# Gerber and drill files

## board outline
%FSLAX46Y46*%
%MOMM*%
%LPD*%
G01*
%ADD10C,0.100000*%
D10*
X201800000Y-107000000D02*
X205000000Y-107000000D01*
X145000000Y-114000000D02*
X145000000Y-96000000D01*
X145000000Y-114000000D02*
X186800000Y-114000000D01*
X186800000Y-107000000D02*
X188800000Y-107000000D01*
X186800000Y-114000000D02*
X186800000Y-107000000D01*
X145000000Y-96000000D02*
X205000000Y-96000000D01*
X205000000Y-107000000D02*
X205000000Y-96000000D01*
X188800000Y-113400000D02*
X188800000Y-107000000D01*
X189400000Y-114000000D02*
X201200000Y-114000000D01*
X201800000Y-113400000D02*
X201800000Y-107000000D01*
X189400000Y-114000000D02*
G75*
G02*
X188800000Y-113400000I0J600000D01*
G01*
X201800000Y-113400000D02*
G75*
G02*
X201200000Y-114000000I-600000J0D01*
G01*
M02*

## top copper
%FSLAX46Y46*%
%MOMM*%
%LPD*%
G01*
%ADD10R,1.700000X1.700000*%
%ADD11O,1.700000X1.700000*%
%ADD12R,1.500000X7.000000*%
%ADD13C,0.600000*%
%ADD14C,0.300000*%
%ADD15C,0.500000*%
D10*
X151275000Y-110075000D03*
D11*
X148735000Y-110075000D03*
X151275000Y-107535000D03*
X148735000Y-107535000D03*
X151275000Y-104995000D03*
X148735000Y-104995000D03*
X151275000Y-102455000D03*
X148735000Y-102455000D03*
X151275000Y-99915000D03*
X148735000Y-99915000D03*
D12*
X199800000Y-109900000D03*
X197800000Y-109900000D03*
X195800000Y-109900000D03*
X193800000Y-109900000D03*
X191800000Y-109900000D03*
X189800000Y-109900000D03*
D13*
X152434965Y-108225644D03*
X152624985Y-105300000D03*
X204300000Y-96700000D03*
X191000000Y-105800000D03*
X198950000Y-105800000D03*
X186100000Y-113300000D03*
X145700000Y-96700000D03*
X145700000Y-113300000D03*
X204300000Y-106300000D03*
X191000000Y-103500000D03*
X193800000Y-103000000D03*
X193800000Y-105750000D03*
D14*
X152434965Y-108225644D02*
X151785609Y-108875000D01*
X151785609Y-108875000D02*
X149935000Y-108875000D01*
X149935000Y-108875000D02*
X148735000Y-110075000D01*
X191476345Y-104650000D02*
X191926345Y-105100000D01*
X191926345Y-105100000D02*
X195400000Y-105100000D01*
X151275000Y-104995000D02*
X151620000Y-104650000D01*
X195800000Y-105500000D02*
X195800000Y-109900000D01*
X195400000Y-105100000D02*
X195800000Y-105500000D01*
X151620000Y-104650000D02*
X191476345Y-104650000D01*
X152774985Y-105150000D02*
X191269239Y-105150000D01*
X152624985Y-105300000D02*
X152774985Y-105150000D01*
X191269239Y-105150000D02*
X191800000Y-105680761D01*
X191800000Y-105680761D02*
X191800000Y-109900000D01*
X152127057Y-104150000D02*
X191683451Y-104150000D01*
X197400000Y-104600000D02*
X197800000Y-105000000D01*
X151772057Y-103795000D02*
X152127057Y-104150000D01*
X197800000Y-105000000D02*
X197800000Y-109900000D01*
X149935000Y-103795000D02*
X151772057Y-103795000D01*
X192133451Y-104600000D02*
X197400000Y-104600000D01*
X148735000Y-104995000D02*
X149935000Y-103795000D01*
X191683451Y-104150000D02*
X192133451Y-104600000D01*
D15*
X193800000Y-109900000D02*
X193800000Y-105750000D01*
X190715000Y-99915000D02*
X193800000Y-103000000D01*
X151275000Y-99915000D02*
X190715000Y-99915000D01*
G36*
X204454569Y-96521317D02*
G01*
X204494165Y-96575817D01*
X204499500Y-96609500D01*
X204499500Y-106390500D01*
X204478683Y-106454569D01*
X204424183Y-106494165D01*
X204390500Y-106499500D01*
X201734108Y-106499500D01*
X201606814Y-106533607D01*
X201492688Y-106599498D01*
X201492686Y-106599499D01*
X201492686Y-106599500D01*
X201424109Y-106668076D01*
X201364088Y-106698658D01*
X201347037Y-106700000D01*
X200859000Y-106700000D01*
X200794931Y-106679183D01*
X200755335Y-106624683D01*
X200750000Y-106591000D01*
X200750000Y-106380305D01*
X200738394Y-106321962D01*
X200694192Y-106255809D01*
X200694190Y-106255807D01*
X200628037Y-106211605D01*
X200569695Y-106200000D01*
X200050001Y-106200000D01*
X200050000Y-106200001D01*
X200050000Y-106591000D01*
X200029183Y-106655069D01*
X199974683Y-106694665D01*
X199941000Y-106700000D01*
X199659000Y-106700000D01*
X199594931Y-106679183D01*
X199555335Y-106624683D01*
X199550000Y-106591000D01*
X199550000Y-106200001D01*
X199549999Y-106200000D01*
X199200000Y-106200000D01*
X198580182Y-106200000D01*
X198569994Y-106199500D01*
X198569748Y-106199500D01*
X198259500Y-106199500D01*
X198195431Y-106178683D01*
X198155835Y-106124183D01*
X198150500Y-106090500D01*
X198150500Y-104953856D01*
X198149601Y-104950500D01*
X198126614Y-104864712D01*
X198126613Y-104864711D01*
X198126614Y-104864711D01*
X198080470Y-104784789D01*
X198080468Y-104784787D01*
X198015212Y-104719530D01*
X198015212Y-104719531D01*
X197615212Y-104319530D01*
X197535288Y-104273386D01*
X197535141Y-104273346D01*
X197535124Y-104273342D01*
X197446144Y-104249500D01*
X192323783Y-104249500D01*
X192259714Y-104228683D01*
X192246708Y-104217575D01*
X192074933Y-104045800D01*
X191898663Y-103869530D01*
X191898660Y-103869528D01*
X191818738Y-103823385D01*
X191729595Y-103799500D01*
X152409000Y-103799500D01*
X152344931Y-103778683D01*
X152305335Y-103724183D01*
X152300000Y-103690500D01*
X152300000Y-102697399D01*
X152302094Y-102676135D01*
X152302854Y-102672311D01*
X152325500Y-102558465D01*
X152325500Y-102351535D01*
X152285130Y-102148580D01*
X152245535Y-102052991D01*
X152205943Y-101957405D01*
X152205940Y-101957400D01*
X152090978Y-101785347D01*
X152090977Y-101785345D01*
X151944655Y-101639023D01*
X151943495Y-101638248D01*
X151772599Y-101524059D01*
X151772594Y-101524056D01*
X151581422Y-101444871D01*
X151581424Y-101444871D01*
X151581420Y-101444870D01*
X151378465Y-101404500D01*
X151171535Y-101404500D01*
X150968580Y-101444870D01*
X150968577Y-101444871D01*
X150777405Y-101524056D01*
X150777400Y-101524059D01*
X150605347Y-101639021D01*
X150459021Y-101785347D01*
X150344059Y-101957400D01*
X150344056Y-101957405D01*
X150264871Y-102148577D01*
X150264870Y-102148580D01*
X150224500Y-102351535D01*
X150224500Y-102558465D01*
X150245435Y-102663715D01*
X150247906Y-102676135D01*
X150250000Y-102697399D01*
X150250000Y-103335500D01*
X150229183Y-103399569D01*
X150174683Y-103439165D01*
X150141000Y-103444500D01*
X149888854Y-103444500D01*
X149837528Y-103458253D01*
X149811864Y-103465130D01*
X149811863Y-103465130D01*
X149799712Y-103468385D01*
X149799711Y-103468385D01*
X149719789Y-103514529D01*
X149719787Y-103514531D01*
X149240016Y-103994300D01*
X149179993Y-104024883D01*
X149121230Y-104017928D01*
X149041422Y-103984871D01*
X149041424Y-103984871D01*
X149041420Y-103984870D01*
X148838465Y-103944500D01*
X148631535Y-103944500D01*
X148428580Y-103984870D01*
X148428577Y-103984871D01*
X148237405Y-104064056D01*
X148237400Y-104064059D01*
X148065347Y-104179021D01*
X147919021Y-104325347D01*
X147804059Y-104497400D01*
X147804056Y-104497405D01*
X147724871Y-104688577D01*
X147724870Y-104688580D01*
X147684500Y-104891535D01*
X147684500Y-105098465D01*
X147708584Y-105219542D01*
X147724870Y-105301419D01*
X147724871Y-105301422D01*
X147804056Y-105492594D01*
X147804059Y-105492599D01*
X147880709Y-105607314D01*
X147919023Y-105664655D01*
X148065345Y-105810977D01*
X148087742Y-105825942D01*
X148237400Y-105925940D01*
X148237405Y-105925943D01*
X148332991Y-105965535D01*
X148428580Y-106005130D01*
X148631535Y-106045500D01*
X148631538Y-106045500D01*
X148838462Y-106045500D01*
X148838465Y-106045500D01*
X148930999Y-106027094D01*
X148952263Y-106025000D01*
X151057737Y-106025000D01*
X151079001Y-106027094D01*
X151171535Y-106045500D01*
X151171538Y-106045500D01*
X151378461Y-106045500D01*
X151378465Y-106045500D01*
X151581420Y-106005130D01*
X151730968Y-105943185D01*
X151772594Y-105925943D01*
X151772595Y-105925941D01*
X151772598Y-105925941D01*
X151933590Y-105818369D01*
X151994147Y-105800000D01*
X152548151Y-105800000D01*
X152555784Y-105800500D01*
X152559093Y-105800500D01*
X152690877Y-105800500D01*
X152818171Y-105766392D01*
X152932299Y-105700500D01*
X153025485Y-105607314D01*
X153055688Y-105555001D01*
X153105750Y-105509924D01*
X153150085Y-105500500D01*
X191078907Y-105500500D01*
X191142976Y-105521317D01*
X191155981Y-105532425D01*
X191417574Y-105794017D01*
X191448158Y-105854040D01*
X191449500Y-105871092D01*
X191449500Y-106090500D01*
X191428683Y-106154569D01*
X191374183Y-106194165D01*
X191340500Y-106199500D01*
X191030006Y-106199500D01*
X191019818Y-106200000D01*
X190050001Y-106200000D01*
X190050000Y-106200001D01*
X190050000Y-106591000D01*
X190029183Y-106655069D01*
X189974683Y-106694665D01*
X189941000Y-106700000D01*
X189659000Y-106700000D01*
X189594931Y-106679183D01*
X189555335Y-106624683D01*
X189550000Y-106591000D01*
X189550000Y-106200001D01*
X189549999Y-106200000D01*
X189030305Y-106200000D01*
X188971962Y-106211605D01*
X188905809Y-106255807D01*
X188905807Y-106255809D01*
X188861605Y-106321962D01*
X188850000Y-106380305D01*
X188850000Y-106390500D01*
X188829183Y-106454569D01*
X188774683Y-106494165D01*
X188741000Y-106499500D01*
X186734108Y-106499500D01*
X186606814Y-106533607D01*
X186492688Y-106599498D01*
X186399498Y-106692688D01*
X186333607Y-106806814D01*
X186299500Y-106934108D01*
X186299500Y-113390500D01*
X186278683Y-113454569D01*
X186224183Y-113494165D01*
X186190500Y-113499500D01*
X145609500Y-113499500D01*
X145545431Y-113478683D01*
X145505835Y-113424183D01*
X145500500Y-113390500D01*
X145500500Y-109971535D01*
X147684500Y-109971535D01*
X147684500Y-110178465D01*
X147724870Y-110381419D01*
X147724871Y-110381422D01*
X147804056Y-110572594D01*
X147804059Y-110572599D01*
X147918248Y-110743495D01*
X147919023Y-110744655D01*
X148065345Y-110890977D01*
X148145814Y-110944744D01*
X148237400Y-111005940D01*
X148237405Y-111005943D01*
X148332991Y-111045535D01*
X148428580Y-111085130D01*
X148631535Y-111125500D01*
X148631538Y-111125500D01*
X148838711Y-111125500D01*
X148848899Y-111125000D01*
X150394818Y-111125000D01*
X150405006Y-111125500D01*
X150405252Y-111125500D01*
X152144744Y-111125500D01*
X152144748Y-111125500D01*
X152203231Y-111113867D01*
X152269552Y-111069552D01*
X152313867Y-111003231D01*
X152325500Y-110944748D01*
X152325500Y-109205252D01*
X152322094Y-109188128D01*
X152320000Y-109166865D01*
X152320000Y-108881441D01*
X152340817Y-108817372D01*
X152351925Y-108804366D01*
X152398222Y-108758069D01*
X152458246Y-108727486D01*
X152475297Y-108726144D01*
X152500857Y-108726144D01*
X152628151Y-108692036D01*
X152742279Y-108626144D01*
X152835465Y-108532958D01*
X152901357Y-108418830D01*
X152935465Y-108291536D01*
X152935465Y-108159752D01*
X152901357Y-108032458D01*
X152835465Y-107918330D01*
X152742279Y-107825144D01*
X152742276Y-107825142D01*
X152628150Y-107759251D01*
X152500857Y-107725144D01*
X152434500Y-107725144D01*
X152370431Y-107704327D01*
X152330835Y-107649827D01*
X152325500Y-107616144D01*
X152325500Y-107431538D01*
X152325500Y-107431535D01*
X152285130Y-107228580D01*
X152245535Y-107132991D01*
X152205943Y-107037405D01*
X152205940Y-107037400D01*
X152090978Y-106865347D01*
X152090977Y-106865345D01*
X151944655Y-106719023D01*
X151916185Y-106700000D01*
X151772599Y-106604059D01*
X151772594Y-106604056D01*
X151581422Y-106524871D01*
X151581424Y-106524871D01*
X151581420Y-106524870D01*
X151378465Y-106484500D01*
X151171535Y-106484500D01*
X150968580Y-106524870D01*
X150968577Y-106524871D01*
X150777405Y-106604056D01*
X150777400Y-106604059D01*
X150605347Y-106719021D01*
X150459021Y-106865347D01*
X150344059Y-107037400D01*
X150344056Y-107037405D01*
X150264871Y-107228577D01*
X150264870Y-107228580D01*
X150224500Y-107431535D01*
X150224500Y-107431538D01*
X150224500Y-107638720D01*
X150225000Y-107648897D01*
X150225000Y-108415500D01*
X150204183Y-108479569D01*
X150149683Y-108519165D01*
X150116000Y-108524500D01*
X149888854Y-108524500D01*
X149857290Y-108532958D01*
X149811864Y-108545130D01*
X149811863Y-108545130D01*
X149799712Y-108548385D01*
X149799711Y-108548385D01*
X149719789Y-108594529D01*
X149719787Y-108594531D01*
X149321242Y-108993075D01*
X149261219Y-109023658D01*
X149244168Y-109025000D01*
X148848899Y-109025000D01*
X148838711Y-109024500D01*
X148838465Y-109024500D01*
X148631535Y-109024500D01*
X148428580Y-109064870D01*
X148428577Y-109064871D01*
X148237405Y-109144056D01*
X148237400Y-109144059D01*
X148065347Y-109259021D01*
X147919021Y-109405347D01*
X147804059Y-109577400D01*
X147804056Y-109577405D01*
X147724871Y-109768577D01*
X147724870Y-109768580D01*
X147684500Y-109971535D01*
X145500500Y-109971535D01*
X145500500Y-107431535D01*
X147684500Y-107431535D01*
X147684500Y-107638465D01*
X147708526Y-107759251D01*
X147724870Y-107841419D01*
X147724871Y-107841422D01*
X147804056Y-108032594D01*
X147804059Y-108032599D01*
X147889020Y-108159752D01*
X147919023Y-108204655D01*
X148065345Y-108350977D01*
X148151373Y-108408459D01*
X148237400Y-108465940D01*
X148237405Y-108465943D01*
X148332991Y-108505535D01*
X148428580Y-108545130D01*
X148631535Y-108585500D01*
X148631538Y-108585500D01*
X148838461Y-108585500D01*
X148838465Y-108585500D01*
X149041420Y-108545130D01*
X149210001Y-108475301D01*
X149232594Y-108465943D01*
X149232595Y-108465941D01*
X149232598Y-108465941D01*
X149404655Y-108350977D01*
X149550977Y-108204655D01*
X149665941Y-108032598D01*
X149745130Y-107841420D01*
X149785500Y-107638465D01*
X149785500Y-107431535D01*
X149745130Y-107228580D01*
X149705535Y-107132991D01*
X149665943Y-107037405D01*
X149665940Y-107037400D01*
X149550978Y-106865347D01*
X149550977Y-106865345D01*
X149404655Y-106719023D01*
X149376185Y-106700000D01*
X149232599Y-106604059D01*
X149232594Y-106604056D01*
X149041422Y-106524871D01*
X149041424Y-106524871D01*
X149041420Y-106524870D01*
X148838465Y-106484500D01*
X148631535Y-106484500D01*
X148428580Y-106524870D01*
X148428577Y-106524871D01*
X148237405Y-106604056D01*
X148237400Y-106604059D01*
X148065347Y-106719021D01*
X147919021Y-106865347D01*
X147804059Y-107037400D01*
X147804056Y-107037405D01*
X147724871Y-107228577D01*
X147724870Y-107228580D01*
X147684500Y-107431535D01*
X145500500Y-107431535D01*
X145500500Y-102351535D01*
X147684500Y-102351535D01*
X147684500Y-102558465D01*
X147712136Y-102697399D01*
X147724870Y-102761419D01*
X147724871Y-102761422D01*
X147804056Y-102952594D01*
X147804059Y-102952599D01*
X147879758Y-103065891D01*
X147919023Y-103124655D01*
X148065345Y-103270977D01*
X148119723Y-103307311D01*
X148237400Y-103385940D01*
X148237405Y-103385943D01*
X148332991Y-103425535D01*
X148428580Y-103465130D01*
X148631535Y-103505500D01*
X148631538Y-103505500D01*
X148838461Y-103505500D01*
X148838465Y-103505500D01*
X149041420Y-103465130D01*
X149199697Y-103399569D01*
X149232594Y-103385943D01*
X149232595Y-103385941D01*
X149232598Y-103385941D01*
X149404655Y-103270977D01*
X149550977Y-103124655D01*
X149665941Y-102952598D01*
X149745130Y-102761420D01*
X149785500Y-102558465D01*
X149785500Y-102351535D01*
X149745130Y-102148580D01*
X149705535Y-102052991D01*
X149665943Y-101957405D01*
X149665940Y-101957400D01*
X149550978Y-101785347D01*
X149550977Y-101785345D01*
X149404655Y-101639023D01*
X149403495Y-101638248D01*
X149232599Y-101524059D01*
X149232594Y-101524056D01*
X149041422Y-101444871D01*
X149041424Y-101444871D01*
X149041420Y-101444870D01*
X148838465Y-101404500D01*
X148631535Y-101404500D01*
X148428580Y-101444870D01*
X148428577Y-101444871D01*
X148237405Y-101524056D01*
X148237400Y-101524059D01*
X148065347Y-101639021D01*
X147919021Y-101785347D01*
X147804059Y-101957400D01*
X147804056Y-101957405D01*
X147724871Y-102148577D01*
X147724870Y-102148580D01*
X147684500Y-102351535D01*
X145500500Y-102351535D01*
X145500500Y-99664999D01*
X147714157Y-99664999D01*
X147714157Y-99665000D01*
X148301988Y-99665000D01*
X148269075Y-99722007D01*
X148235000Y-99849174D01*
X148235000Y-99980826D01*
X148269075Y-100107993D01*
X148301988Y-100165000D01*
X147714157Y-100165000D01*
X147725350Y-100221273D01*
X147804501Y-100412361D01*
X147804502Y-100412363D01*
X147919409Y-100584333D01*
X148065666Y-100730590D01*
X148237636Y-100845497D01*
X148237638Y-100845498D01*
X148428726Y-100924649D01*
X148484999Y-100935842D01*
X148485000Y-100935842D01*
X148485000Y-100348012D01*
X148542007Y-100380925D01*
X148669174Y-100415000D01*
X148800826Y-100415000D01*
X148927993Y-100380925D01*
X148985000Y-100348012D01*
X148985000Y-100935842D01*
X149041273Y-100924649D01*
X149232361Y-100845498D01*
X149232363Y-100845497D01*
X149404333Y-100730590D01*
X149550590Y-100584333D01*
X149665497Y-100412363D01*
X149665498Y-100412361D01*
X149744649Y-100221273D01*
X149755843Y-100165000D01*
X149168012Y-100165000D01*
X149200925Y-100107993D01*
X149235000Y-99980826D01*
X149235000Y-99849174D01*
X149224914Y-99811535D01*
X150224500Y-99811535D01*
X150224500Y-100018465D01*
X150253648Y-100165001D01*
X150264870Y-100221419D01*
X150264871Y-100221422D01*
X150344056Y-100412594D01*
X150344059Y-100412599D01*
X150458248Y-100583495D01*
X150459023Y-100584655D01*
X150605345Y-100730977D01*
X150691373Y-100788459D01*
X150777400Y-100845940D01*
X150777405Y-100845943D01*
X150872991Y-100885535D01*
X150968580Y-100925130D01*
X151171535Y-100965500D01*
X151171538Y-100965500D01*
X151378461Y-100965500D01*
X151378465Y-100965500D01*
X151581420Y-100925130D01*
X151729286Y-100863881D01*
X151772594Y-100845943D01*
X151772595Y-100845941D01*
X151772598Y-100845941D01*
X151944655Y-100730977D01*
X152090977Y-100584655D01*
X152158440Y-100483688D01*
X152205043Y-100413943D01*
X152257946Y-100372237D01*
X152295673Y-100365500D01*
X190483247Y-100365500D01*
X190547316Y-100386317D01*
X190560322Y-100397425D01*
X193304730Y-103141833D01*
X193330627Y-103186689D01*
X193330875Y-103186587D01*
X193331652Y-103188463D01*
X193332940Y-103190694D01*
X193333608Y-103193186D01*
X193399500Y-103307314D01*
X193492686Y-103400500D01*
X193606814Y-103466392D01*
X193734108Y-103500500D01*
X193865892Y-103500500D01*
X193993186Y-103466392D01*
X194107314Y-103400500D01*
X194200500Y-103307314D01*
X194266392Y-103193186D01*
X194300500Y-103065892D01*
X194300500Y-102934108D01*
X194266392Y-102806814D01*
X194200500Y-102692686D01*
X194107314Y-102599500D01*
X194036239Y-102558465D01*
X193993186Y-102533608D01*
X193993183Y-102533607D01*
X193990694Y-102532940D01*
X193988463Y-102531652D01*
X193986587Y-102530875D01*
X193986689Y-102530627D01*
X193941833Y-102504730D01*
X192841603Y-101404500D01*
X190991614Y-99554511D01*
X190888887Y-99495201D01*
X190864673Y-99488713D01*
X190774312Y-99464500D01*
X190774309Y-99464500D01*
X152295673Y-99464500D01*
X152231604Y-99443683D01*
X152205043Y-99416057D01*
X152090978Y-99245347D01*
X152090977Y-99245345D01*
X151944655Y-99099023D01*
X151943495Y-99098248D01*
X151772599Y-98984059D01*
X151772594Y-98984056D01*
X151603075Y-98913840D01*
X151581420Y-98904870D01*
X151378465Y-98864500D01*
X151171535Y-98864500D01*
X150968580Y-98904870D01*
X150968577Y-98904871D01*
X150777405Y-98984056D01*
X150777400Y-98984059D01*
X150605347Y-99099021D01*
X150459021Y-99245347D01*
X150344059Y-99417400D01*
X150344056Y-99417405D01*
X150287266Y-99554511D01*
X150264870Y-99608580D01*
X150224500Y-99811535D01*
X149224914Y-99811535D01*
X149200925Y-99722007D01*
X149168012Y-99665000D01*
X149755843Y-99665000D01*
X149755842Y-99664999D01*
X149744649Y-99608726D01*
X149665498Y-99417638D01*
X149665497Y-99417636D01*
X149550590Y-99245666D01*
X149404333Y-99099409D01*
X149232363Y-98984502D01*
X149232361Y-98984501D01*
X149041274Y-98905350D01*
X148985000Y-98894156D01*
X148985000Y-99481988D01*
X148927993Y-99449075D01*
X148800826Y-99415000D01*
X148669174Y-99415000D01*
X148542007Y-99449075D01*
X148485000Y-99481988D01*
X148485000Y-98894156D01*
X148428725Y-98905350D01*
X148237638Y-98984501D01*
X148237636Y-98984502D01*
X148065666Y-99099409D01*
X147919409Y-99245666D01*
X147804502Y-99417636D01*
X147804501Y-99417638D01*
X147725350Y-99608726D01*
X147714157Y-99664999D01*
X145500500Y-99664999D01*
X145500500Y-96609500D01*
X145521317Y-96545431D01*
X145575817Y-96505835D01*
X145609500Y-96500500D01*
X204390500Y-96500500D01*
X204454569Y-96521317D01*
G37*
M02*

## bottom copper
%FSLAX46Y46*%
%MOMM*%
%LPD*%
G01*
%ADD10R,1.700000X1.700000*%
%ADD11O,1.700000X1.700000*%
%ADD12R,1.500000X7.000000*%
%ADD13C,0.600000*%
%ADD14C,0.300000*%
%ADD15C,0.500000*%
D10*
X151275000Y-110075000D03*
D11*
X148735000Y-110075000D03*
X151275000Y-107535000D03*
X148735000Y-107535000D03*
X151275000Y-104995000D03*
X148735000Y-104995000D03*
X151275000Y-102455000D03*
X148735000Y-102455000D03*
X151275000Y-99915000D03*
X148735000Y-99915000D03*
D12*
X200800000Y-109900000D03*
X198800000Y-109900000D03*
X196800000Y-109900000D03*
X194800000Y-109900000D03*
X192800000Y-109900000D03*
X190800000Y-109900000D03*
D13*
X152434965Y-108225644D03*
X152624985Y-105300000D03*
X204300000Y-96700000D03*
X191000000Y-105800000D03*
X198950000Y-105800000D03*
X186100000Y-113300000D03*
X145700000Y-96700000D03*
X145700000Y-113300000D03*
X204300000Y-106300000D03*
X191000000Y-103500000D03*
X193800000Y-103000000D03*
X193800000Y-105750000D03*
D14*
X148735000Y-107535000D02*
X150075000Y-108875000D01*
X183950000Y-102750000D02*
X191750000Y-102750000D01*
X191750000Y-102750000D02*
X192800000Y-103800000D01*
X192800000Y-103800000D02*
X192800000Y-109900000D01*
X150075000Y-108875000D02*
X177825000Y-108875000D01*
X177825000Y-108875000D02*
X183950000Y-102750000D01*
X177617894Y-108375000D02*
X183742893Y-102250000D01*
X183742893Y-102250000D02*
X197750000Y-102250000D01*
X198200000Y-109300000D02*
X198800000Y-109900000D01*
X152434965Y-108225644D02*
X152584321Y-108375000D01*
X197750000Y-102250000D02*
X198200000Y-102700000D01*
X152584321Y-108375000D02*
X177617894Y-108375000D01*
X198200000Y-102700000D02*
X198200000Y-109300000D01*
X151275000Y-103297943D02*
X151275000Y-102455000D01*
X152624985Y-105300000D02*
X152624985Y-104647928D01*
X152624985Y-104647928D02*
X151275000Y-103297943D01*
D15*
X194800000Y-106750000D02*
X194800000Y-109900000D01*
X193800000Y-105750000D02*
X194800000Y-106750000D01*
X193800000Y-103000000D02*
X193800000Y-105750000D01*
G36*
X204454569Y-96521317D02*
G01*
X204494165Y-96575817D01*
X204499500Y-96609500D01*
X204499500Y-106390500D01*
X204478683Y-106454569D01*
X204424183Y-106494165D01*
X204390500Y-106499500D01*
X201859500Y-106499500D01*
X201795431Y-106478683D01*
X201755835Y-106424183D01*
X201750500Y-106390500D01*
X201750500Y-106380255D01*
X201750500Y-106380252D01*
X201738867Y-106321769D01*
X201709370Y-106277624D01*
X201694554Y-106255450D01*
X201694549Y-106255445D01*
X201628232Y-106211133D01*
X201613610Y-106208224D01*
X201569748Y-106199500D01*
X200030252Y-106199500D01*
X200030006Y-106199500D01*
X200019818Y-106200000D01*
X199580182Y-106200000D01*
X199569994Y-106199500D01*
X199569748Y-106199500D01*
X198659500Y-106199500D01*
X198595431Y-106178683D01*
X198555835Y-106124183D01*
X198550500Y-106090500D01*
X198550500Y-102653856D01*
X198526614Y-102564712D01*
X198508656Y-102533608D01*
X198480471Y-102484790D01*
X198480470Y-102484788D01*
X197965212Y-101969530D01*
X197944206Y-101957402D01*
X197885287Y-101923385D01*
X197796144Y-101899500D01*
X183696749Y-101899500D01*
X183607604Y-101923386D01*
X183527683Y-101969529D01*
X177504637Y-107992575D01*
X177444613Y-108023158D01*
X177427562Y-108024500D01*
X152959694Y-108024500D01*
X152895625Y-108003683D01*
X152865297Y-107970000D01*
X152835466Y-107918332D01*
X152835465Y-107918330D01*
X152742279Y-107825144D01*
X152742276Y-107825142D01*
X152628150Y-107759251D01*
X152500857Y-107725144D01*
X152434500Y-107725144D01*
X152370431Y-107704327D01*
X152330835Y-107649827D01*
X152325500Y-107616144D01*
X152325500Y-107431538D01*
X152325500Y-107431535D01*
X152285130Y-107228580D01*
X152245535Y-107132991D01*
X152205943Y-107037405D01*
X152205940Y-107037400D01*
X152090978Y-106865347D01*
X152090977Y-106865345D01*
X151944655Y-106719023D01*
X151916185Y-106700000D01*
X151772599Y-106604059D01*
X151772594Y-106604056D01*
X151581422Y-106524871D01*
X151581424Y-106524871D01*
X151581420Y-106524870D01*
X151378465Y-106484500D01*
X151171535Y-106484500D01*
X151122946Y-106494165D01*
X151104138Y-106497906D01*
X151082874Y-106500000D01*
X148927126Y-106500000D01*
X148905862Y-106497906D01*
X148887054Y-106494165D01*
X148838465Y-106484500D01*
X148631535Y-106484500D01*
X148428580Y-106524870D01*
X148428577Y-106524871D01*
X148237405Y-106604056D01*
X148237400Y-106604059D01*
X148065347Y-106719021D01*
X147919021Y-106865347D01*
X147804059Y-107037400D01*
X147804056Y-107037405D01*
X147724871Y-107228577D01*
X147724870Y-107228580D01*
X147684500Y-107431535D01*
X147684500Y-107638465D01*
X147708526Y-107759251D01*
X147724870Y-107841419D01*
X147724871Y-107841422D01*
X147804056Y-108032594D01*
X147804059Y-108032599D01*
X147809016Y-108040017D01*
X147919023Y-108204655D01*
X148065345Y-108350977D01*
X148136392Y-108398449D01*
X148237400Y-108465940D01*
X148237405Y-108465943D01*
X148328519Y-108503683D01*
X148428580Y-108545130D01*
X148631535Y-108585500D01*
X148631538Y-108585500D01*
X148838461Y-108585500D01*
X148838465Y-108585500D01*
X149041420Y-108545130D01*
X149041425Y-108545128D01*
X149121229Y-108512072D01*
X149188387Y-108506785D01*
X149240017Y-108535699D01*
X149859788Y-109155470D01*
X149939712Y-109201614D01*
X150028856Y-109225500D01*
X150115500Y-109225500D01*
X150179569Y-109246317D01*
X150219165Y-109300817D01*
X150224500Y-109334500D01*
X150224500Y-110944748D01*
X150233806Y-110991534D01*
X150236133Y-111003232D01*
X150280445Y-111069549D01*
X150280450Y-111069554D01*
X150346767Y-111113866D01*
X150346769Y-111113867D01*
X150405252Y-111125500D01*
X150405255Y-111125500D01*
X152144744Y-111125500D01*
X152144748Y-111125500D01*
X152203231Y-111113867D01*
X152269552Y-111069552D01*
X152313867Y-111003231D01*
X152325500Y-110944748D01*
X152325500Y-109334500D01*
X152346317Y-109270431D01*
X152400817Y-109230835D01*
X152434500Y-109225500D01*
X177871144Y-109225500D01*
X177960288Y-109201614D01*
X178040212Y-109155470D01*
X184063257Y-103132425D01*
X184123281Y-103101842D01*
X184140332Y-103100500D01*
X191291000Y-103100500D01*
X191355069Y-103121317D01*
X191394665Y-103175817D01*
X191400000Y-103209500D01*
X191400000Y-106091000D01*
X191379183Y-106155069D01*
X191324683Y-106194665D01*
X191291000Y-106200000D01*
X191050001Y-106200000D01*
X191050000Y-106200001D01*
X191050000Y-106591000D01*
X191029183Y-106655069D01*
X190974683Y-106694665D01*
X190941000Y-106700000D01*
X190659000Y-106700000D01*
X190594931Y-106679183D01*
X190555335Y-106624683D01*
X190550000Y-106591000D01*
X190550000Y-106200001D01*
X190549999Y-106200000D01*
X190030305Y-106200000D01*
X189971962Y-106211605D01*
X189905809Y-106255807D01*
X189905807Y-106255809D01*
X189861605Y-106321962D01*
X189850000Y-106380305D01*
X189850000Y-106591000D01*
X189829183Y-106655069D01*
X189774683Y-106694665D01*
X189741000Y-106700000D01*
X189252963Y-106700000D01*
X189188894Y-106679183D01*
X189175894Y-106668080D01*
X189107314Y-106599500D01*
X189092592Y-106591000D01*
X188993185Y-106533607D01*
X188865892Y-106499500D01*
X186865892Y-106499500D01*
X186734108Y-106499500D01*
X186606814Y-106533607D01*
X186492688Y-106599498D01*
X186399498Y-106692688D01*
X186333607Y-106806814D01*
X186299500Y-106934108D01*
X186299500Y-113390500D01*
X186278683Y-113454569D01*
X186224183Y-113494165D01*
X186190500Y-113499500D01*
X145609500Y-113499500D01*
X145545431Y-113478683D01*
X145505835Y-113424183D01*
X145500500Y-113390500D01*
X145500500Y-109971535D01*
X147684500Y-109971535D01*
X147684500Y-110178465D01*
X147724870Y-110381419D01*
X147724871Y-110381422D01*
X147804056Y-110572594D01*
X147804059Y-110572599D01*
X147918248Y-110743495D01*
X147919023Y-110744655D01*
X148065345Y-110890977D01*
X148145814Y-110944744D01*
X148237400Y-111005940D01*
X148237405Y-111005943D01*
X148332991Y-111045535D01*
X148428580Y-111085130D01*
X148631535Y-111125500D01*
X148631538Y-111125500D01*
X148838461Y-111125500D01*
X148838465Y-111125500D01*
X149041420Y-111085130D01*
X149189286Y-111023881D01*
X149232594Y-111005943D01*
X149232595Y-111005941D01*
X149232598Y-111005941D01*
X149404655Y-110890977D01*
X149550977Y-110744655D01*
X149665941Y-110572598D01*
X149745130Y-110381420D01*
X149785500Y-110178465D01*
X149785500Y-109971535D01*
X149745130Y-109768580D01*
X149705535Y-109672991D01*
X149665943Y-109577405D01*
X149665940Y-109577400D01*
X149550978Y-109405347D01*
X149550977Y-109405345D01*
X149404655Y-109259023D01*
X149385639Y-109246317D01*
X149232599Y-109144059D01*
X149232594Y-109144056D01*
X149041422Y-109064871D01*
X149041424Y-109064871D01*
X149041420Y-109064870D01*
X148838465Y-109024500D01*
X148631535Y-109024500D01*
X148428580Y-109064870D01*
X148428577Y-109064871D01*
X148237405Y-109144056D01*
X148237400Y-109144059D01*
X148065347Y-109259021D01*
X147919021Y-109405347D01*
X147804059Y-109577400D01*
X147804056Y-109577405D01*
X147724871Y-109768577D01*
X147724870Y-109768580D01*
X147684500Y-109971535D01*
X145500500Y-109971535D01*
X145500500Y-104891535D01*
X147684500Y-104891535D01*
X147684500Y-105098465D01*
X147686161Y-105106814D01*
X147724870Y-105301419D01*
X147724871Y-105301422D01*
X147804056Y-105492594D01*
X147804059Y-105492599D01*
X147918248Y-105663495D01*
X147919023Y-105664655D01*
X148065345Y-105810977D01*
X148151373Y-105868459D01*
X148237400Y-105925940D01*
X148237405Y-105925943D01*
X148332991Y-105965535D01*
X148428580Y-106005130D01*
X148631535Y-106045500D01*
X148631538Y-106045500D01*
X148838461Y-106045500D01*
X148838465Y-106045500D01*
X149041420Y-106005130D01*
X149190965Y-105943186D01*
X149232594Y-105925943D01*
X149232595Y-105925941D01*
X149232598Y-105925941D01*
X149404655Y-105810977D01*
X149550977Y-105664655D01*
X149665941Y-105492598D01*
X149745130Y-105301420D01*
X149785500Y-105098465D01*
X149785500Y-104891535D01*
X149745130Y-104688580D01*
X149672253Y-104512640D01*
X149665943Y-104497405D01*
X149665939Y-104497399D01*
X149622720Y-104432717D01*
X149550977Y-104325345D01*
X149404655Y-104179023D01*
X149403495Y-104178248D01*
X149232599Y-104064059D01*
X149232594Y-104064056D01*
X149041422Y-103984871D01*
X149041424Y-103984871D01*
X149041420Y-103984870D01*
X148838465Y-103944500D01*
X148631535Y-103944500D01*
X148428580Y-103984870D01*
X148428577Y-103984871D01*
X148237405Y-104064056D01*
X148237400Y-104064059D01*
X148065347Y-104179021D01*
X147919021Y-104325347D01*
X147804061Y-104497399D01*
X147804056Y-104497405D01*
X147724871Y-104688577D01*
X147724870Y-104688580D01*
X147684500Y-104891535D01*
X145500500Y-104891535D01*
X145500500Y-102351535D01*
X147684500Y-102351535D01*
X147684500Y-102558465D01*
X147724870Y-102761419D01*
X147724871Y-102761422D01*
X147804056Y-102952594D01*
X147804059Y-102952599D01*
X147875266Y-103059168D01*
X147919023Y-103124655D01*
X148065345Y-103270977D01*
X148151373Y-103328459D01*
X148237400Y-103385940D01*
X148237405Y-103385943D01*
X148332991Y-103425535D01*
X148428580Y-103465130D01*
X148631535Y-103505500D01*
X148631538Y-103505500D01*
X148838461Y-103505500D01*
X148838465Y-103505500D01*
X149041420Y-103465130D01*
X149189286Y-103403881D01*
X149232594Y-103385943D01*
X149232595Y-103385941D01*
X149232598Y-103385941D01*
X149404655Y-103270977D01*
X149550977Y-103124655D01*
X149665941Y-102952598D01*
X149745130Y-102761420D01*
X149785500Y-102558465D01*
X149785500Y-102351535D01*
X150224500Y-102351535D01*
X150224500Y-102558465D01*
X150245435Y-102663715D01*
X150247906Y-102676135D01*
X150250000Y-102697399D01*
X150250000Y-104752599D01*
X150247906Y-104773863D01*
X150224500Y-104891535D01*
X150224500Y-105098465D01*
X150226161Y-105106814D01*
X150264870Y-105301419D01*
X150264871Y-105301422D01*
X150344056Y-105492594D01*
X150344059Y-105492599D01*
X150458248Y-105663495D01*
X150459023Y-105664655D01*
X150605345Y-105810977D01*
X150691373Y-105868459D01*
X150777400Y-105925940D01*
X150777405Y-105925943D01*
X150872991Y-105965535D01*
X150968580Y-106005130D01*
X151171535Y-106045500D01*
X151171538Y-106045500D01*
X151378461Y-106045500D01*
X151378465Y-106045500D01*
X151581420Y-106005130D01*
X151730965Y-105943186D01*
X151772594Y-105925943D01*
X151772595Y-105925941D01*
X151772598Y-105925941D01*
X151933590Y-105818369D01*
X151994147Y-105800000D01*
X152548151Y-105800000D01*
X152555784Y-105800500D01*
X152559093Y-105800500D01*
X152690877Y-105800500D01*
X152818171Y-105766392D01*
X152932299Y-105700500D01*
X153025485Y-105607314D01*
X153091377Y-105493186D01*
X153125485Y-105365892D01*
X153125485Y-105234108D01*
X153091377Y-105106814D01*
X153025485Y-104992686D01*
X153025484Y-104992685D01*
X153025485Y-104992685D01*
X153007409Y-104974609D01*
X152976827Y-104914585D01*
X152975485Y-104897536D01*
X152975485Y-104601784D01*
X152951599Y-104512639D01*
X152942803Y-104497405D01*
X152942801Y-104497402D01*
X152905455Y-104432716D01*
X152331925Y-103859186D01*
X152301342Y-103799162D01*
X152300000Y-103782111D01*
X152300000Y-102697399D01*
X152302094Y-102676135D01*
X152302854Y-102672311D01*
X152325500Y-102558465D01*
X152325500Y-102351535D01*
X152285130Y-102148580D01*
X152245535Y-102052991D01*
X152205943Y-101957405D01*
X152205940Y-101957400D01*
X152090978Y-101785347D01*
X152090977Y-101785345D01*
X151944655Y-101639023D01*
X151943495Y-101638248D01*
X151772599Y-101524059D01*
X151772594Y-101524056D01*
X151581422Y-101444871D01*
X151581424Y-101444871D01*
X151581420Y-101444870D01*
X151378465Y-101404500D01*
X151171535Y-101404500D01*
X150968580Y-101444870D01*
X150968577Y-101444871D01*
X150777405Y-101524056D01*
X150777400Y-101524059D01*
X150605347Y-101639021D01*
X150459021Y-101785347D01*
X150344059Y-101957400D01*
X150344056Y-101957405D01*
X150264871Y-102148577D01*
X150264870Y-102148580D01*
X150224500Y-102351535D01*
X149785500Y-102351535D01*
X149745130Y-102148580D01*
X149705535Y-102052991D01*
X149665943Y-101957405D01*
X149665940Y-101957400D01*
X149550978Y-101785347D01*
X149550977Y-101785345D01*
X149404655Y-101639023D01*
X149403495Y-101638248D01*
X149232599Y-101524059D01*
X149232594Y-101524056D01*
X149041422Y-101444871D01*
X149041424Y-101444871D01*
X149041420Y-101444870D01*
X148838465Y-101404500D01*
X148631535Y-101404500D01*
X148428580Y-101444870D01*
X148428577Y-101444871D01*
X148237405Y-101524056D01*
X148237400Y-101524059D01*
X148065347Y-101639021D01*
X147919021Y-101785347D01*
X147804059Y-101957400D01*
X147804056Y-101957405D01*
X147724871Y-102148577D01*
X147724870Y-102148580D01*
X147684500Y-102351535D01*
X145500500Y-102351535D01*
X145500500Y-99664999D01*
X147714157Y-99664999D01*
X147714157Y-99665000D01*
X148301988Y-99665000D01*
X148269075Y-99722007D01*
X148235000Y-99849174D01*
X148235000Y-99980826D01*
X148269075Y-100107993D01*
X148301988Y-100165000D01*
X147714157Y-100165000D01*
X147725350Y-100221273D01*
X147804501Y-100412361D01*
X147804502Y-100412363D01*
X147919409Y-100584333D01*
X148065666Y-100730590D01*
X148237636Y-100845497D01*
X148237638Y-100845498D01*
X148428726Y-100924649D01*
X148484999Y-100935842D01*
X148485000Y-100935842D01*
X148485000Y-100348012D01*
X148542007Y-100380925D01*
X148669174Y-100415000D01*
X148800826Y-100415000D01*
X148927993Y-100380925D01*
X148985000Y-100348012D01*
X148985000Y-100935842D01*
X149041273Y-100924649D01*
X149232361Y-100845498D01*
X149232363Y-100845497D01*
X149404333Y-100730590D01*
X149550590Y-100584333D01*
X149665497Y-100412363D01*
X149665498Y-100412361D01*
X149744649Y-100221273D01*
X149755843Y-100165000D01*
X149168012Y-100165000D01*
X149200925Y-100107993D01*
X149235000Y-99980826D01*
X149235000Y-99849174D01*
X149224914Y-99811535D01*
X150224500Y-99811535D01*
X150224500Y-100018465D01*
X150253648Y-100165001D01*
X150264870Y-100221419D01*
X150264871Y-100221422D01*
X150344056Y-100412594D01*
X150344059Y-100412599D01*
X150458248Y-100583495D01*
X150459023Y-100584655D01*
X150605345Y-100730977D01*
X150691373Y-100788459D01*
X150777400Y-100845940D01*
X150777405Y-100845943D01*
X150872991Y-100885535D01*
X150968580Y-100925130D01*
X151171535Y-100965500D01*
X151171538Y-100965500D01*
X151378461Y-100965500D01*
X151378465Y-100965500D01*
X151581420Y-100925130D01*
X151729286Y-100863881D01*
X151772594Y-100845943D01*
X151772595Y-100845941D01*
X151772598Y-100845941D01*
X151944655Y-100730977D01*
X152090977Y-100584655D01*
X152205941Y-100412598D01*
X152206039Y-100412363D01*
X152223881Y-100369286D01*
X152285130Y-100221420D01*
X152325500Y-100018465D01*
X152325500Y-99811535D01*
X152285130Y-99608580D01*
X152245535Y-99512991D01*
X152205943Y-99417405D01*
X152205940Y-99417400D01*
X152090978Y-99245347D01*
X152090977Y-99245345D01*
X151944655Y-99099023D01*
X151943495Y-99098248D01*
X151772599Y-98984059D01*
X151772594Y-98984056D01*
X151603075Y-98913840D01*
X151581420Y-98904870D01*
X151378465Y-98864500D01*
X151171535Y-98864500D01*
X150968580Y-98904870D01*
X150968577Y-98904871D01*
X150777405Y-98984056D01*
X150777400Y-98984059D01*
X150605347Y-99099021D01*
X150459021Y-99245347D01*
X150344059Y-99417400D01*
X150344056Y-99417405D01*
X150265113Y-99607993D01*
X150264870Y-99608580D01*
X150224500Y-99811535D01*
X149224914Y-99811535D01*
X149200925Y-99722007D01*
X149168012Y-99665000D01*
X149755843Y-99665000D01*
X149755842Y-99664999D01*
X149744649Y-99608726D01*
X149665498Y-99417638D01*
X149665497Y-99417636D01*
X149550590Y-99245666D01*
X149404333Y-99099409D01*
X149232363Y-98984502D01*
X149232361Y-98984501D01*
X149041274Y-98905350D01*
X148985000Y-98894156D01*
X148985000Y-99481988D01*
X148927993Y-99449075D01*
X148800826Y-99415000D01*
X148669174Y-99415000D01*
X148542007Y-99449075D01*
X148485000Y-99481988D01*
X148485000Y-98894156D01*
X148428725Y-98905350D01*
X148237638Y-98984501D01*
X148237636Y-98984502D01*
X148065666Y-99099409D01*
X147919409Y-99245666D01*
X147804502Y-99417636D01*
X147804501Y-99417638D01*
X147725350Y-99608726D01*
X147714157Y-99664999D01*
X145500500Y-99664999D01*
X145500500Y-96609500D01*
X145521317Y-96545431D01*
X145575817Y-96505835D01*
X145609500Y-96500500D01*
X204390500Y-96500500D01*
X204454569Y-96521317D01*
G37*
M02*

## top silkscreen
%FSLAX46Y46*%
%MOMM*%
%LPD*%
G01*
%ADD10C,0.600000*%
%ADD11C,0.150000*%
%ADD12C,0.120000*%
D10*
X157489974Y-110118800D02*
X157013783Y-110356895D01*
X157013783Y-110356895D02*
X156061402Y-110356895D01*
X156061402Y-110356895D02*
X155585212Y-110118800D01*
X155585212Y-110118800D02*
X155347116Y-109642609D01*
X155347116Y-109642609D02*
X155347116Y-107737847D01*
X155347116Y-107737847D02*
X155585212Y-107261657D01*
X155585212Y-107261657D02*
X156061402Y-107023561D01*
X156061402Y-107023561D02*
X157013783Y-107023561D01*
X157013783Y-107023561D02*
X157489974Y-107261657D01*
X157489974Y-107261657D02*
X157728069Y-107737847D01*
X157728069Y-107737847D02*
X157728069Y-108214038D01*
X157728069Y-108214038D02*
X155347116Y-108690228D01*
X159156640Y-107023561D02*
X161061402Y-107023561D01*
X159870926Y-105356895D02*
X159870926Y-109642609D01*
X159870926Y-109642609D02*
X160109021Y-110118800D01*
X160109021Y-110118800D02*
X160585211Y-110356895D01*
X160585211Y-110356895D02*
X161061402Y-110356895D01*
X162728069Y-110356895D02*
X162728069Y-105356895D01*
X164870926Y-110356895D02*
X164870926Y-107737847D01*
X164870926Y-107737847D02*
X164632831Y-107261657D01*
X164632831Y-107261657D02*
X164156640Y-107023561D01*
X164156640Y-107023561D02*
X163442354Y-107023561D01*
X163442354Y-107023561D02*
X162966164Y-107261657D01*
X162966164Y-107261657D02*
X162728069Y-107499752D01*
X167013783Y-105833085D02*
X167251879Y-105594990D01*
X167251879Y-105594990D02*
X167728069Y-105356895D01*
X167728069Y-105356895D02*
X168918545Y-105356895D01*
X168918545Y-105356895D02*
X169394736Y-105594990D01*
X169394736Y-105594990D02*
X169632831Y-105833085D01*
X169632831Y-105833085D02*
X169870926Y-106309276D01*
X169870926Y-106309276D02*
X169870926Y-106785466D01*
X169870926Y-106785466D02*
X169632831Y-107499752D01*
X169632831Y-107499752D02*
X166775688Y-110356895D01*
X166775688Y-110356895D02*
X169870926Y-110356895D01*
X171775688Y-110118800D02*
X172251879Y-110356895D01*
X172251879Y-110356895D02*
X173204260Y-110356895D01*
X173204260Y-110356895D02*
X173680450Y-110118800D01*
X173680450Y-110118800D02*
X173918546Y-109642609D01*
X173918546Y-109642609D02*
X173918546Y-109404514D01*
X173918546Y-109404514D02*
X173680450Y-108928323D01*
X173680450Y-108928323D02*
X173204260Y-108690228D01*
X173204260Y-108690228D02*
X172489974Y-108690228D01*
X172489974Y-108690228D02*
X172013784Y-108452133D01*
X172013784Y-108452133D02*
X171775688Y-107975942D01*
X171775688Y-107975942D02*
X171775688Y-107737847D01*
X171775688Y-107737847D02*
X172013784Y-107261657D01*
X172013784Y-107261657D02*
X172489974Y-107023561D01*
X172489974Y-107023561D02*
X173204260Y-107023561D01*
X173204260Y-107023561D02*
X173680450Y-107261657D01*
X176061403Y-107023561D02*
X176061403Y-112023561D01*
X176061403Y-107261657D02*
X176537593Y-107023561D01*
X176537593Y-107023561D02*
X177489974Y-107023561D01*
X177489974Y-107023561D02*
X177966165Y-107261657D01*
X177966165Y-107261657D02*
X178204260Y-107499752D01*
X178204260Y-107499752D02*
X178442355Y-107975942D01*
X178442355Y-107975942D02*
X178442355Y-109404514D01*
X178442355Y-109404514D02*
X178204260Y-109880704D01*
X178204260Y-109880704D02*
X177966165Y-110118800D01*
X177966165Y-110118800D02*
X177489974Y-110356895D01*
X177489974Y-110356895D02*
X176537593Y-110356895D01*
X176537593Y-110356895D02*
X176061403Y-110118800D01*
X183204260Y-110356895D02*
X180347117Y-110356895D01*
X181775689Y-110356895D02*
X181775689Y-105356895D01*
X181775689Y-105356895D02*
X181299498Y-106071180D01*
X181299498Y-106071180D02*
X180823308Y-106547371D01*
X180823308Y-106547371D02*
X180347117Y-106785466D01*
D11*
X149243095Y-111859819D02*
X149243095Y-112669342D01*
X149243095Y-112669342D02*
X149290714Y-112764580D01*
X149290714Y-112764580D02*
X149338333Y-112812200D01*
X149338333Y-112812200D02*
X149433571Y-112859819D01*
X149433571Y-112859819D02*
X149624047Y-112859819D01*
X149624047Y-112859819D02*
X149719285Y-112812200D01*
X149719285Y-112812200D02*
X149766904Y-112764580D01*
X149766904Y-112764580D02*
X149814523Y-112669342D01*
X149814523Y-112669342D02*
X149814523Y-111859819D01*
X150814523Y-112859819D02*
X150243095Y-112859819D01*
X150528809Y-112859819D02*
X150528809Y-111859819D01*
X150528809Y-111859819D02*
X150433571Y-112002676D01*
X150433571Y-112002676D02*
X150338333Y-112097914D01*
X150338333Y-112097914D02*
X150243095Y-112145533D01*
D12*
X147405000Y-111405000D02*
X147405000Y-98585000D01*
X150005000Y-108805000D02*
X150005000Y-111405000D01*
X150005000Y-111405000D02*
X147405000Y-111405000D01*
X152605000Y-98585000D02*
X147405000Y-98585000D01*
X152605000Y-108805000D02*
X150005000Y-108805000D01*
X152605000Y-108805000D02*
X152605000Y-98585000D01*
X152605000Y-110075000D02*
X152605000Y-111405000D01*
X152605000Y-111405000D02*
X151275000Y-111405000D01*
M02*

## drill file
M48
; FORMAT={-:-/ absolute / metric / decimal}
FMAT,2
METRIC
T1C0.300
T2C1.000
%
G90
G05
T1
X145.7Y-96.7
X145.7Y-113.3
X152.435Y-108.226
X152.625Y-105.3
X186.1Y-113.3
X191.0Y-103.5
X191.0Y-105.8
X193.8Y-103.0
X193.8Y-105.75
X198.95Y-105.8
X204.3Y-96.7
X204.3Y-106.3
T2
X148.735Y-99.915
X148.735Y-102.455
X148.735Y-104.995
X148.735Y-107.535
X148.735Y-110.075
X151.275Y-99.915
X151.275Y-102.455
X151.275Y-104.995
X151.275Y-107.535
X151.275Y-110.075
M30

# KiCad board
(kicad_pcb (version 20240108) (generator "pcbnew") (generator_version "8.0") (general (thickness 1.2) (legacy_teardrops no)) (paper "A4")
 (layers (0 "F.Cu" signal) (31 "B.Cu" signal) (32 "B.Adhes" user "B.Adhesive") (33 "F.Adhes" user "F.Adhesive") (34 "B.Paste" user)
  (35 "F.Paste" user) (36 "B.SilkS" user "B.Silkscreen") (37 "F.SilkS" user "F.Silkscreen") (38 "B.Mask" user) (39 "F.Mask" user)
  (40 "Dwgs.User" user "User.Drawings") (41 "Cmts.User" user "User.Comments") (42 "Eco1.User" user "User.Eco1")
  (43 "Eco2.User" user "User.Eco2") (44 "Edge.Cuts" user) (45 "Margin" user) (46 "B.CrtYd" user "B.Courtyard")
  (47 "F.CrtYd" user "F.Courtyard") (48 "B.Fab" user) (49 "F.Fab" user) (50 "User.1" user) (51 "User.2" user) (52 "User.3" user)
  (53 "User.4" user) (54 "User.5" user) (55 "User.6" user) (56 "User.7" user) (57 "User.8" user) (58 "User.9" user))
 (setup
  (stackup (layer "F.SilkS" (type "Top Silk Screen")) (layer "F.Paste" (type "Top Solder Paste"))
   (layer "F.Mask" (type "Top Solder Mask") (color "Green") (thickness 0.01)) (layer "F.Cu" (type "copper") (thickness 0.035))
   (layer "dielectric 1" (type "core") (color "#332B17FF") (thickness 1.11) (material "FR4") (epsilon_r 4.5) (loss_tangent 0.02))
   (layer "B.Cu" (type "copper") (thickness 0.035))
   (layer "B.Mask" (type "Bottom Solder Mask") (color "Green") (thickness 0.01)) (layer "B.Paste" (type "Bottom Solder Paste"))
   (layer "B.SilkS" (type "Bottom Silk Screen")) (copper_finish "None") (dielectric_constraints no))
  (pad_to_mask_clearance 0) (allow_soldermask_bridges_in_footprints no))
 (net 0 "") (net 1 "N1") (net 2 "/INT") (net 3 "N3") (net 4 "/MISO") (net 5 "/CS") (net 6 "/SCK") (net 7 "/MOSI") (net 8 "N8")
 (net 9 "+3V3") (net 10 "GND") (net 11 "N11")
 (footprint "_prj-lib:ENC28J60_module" (layer "F.Cu") (at 151.275 110.075 180)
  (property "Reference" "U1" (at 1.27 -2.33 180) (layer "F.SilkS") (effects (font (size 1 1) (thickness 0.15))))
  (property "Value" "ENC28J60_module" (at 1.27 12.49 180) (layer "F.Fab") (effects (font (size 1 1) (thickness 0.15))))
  (fp_line (start 3.87 -1.33) (end 3.87 11.49) (stroke (width 0.12) (type solid)) (layer "F.SilkS"))
  (fp_line (start 1.27 1.27) (end 1.27 -1.33) (stroke (width 0.12) (type solid)) (layer "F.SilkS"))
  (fp_line (start 1.27 -1.33) (end 3.87 -1.33) (stroke (width 0.12) (type solid)) (layer "F.SilkS"))
  (fp_line (start -1.33 11.49) (end 3.87 11.49) (stroke (width 0.12) (type solid)) (layer "F.SilkS"))
  (fp_line (start -1.33 1.27) (end 1.27 1.27) (stroke (width 0.12) (type solid)) (layer "F.SilkS"))
  (fp_line (start -1.33 1.27) (end -1.33 11.49) (stroke (width 0.12) (type solid)) (layer "F.SilkS"))
  (fp_line (start -1.33 0) (end -1.33 -1.33) (stroke (width 0.12) (type solid)) (layer "F.SilkS"))
  (fp_line (start -1.33 -1.33) (end 0 -1.33) (stroke (width 0.12) (type solid)) (layer "F.SilkS"))
  (pad "1" thru_hole rect (at 0 0 180) (size 1.7 1.7) (drill 1) (layers "*.Cu" "*.Mask") (remove_unused_layers no) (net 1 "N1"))
  (pad "2" thru_hole oval (at 2.54 0 180) (size 1.7 1.7) (drill 1) (layers "*.Cu" "*.Mask") (remove_unused_layers no) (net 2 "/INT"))
  (pad "3" thru_hole oval (at 0 2.54 180) (size 1.7 1.7) (drill 1) (layers "*.Cu" "*.Mask") (remove_unused_layers no) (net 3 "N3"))
  (pad "4" thru_hole oval (at 2.54 2.54 180) (size 1.7 1.7) (drill 1) (layers "*.Cu" "*.Mask") (remove_unused_layers no) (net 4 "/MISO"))
  (pad "5" thru_hole oval (at 0 5.08 180) (size 1.7 1.7) (drill 1) (layers "*.Cu" "*.Mask") (remove_unused_layers no) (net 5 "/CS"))
  (pad "6" thru_hole oval (at 2.54 5.08 180) (size 1.7 1.7) (drill 1) (layers "*.Cu" "*.Mask") (remove_unused_layers no) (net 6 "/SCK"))
  (pad "7" thru_hole oval (at 0 7.62 180) (size 1.7 1.7) (drill 1) (layers "*.Cu" "*.Mask") (remove_unused_layers no) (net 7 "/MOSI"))
  (pad "8" thru_hole oval (at 2.54 7.62 180) (size 1.7 1.7) (drill 1) (layers "*.Cu" "*.Mask") (remove_unused_layers no) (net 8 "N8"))
  (pad "9" thru_hole oval (at 0 10.16 180) (size 1.7 1.7) (drill 1) (layers "*.Cu" "*.Mask") (remove_unused_layers no) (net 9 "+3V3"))
  (pad "10" thru_hole oval (at 2.54 10.16 180) (size 1.7 1.7) (drill 1) (layers "*.Cu" "*.Mask") (remove_unused_layers no) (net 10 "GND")))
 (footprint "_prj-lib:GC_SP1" (layer "B.Cu") (at 195.3 107 180)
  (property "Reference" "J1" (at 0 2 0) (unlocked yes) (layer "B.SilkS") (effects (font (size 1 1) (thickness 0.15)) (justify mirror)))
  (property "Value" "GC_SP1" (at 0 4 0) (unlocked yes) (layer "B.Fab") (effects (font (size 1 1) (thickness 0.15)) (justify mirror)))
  (fp_line (start 6.5 -6.4) (end 6.5 0) (stroke (width 0.1) (type solid)) (layer "Edge.Cuts"))
  (fp_line (start 5.9 -7) (end -5.9 -7) (stroke (width 0.1) (type solid)) (layer "Edge.Cuts"))
  (fp_line (start -6.5 -6.4) (end -6.5 0) (stroke (width 0.1) (type solid)) (layer "Edge.Cuts"))
  (fp_arc (start 5.9 -7) (mid 6.324264 -6.824264) (end 6.5 -6.4) (stroke (width 0.1) (type solid)) (layer "Edge.Cuts"))
  (fp_arc (start -6.5 -6.4) (mid -6.324264 -6.824264) (end -5.9 -7) (stroke (width 0.1) (type solid)) (layer "Edge.Cuts"))
  (pad "1" smd rect (at -5.5 -2.9 180) (size 1.5 7) (layers "B.Cu" "B.Mask") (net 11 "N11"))
  (pad "2" smd rect (at -4.5 -2.9 180) (size 1.5 7) (layers "F.Cu" "F.Mask") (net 10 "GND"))
  (pad "3" smd rect (at -3.5 -2.9 180) (size 1.5 7) (layers "B.Cu" "B.Mask") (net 2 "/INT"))
  (pad "4" smd rect (at -2.5 -2.9 180) (size 1.5 7) (layers "F.Cu" "F.Mask") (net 6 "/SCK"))
  (pad "5" smd rect (at -1.5 -2.9 180) (size 1.5 7) (layers "B.Cu" "B.Mask"))
  (pad "6" smd rect (at -0.5 -2.9 180) (size 1.5 7) (layers "F.Cu" "F.Mask") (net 5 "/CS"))
  (pad "7" smd rect (at 0.5 -2.9 180) (size 1.5 7) (layers "B.Cu" "B.Mask") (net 9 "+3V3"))
  (pad "8" smd rect (at 1.5 -2.9 180) (size 1.5 7) (layers "F.Cu" "F.Mask") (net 9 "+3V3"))
  (pad "9" smd rect (at 2.5 -2.9 180) (size 1.5 7) (layers "B.Cu" "B.Mask") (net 4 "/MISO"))
  (pad "10" smd rect (at 3.5 -2.9 180) (size 1.5 7) (layers "F.Cu" "F.Mask") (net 7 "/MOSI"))
  (pad "11" smd rect (at 4.5 -2.9 180) (size 1.5 7) (layers "B.Cu" "B.Mask") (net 10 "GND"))
  (pad "12" smd rect (at 5.5 -2.9 180) (size 1.5 7) (layers "F.Cu" "F.Mask") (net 10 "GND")))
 (gr_line (start 201.8 107) (end 205 107) (stroke (width 0.1) (type solid)) (layer "Edge.Cuts"))
 (gr_line (start 145 114) (end 145 96) (stroke (width 0.1) (type default)) (layer "Edge.Cuts"))
 (gr_line (start 145 114) (end 186.8 114) (stroke (width 0.1) (type default)) (layer "Edge.Cuts"))
 (gr_line (start 186.8 107) (end 188.8 107) (stroke (width 0.1) (type solid)) (layer "Edge.Cuts"))
 (gr_line (start 186.8 114) (end 186.8 107) (stroke (width 0.1) (type solid)) (layer "Edge.Cuts"))
 (gr_line (start 145 96) (end 205 96) (stroke (width 0.1) (type default)) (layer "Edge.Cuts"))
 (gr_line (start 205 107) (end 205 96) (stroke (width 0.1) (type default)) (layer "Edge.Cuts"))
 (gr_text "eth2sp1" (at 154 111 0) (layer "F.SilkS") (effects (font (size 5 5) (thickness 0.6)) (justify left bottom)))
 (segment (start 148.735 107.535) (end 150.075 108.875) (width 0.3) (layer "B.Cu") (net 4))
 (segment (start 183.95 102.75) (end 191.75 102.75) (width 0.3) (layer "B.Cu") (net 4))
 (segment (start 191.75 102.75) (end 192.8 103.8) (width 0.3) (layer "B.Cu") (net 4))
 (segment (start 192.8 103.8) (end 192.8 109.9) (width 0.3) (layer "B.Cu") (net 4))
 (segment (start 150.075 108.875) (end 177.825 108.875) (width 0.3) (layer "B.Cu") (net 4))
 (segment (start 177.825 108.875) (end 183.95 102.75) (width 0.3) (layer "B.Cu") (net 4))
 (segment (start 152.434965 108.225644) (end 151.785609 108.875) (width 0.3) (layer "F.Cu") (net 2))
 (segment (start 151.785609 108.875) (end 149.935 108.875) (width 0.3) (layer "F.Cu") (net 2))
 (segment (start 149.935 108.875) (end 148.735 110.075) (width 0.3) (layer "F.Cu") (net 2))
 (via (at 152.434965 108.225644) (size 0.6) (drill 0.3) (layers "F.Cu" "B.Cu") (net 2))
 (segment (start 177.617894 108.375) (end 183.742893 102.25) (width 0.3) (layer "B.Cu") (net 2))
 (segment (start 183.742893 102.25) (end 197.75 102.25) (width 0.3) (layer "B.Cu") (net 2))
 (segment (start 198.2 109.3) (end 198.8 109.9) (width 0.3) (layer "B.Cu") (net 2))
 (segment (start 152.434965 108.225644) (end 152.584321 108.375) (width 0.3) (layer "B.Cu") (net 2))
 (segment (start 197.75 102.25) (end 198.2 102.7) (width 0.3) (layer "B.Cu") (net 2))
 (segment (start 152.584321 108.375) (end 177.617894 108.375) (width 0.3) (layer "B.Cu") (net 2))
 (segment (start 198.2 102.7) (end 198.2 109.3) (width 0.3) (layer "B.Cu") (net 2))
 (segment (start 191.476345 104.65) (end 191.926345 105.1) (width 0.3) (layer "F.Cu") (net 5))
 (segment (start 191.926345 105.1) (end 195.4 105.1) (width 0.3) (layer "F.Cu") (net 5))
 (segment (start 151.275 104.995) (end 151.62 104.65) (width 0.3) (layer "F.Cu") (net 5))
 (segment (start 195.8 105.5) (end 195.8 109.9) (width 0.3) (layer "F.Cu") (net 5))
 (segment (start 195.4 105.1) (end 195.8 105.5) (width 0.3) (layer "F.Cu") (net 5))
 (segment (start 151.62 104.65) (end 191.476345 104.65) (width 0.3) (layer "F.Cu") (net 5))
 (segment (start 152.774985 105.15) (end 191.269239 105.15) (width 0.3) (layer "F.Cu") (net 7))
 (segment (start 152.624985 105.3) (end 152.774985 105.15) (width 0.3) (layer "F.Cu") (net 7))
 (segment (start 191.269239 105.15) (end 191.8 105.680761) (width 0.3) (layer "F.Cu") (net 7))
 (segment (start 191.8 105.680761) (end 191.8 109.9) (width 0.3) (layer "F.Cu") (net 7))
 (via (at 152.624985 105.3) (size 0.6) (drill 0.3) (layers "F.Cu" "B.Cu") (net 7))
 (segment (start 151.275 103.297943) (end 151.275 102.455) (width 0.3) (layer "B.Cu") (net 7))
 (segment (start 152.624985 105.3) (end 152.624985 104.647928) (width 0.3) (layer "B.Cu") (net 7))
 (segment (start 152.624985 104.647928) (end 151.275 103.297943) (width 0.3) (layer "B.Cu") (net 7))
 (segment (start 152.127057 104.15) (end 191.683451 104.15) (width 0.3) (layer "F.Cu") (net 6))
 (segment (start 197.4 104.6) (end 197.8 105) (width 0.3) (layer "F.Cu") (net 6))
 (segment (start 151.772057 103.795) (end 152.127057 104.15) (width 0.3) (layer "F.Cu") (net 6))
 (segment (start 197.8 105) (end 197.8 109.9) (width 0.3) (layer "F.Cu") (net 6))
 (segment (start 149.935 103.795) (end 151.772057 103.795) (width 0.3) (layer "F.Cu") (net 6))
 (segment (start 192.133451 104.6) (end 197.4 104.6) (width 0.3) (layer "F.Cu") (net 6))
 (segment (start 148.735 104.995) (end 149.935 103.795) (width 0.3) (layer "F.Cu") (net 6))
 (segment (start 191.683451 104.15) (end 192.133451 104.6) (width 0.3) (layer "F.Cu") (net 6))
 (via (at 204.3 96.7) (size 0.6) (drill 0.3) (layers "F.Cu" "B.Cu") (free yes) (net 10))
 (via (at 191 105.8) (size 0.6) (drill 0.3) (layers "F.Cu" "B.Cu") (free yes) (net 10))
 (via (at 198.95 105.8) (size 0.6) (drill 0.3) (layers "F.Cu" "B.Cu") (free yes) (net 10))
 (via (at 186.1 113.3) (size 0.6) (drill 0.3) (layers "F.Cu" "B.Cu") (free yes) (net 10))
 (via (at 145.7 96.7) (size 0.6) (drill 0.3) (layers "F.Cu" "B.Cu") (free yes) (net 10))
 (via (at 145.7 113.3) (size 0.6) (drill 0.3) (layers "F.Cu" "B.Cu") (free yes) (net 10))
 (via (at 204.3 106.3) (size 0.6) (drill 0.3) (layers "F.Cu" "B.Cu") (free yes) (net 10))
 (via (at 191 103.5) (size 0.6) (drill 0.3) (layers "F.Cu" "B.Cu") (free yes) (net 10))
 (segment (start 193.8 109.9) (end 193.8 105.75) (width 0.5) (layer "F.Cu") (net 9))
 (segment (start 190.715 99.915) (end 193.8 103) (width 0.5) (layer "F.Cu") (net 9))
 (segment (start 151.275 99.915) (end 190.715 99.915) (width 0.5) (layer "F.Cu") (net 9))
 (via (at 193.8 103) (size 0.6) (drill 0.3) (layers "F.Cu" "B.Cu") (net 9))
 (via (at 193.8 105.75) (size 0.6) (drill 0.3) (layers "F.Cu" "B.Cu") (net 9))
 (segment (start 194.8 106.75) (end 194.8 109.9) (width 0.5) (layer "B.Cu") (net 9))
 (segment (start 193.8 105.75) (end 194.8 106.75) (width 0.5) (layer "B.Cu") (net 9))
 (segment (start 193.8 103) (end 193.8 105.75) (width 0.5) (layer "B.Cu") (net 9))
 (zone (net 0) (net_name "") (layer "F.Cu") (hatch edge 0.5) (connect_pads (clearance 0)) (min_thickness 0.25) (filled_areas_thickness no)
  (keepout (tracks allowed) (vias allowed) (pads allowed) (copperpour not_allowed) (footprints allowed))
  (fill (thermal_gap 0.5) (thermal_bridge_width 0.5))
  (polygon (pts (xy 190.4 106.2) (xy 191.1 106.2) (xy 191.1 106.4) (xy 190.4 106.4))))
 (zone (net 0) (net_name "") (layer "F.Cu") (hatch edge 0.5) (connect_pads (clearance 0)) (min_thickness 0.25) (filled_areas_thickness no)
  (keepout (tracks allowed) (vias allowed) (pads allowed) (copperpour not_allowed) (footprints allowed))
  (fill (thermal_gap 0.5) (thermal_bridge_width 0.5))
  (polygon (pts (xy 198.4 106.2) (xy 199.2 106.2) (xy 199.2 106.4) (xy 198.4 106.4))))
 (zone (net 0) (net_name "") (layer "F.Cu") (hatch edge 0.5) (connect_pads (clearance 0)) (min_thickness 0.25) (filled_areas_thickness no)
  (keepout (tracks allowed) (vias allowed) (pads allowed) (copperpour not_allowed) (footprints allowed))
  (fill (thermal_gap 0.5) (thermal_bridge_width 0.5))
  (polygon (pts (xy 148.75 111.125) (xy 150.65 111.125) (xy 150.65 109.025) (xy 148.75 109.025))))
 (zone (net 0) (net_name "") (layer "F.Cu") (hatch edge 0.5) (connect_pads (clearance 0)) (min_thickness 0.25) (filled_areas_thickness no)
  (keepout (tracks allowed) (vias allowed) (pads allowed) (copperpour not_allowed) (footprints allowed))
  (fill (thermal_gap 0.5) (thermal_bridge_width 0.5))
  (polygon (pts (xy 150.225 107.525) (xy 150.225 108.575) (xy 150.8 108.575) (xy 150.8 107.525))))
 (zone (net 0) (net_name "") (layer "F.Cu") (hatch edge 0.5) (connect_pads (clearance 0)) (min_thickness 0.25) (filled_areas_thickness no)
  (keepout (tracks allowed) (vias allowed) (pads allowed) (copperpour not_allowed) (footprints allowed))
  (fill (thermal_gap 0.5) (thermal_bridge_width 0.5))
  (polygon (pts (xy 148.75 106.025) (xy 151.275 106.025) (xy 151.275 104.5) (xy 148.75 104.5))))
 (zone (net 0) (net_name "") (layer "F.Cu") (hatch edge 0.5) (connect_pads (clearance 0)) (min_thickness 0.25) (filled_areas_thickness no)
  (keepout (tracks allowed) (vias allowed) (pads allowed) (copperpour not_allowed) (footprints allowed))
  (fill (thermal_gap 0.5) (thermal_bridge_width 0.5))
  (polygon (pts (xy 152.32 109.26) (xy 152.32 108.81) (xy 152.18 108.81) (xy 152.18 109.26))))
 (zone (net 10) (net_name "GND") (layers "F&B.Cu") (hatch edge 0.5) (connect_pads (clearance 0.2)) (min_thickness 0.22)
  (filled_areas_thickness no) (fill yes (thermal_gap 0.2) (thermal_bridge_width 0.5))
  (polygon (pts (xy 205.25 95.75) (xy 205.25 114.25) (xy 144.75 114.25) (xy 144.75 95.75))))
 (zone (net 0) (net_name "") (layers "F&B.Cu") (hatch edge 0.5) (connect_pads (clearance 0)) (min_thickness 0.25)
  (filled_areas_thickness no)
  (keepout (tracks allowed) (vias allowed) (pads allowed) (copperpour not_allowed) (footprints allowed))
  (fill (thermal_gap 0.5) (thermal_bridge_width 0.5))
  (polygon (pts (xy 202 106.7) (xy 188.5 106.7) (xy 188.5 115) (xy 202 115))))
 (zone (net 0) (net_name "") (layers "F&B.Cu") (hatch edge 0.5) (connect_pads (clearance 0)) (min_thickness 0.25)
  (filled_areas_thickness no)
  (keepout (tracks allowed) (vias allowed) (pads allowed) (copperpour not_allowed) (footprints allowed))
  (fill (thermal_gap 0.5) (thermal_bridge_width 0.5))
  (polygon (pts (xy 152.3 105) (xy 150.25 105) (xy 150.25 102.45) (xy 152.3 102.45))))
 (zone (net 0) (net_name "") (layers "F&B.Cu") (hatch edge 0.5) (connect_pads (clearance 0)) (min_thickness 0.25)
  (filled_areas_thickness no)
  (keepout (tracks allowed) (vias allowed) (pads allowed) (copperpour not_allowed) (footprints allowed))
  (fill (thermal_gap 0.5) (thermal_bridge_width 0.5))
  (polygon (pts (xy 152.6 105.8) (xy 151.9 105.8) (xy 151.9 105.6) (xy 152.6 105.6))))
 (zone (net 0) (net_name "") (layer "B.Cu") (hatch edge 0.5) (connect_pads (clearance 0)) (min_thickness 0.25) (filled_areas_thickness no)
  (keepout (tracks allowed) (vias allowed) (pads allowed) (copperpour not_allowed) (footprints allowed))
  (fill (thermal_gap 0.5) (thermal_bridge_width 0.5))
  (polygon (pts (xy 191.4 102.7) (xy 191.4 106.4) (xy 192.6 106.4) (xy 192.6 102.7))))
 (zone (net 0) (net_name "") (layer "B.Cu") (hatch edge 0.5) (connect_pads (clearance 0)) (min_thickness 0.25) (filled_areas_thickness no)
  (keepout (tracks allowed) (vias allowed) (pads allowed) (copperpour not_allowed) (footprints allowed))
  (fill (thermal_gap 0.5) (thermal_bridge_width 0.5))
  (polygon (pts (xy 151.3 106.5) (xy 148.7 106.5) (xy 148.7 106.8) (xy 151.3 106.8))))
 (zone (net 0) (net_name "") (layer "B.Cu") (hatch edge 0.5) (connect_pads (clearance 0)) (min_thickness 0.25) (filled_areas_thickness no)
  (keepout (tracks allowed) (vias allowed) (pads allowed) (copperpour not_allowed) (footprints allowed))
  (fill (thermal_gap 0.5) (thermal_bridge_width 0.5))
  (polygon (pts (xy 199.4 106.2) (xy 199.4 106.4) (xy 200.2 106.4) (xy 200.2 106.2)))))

